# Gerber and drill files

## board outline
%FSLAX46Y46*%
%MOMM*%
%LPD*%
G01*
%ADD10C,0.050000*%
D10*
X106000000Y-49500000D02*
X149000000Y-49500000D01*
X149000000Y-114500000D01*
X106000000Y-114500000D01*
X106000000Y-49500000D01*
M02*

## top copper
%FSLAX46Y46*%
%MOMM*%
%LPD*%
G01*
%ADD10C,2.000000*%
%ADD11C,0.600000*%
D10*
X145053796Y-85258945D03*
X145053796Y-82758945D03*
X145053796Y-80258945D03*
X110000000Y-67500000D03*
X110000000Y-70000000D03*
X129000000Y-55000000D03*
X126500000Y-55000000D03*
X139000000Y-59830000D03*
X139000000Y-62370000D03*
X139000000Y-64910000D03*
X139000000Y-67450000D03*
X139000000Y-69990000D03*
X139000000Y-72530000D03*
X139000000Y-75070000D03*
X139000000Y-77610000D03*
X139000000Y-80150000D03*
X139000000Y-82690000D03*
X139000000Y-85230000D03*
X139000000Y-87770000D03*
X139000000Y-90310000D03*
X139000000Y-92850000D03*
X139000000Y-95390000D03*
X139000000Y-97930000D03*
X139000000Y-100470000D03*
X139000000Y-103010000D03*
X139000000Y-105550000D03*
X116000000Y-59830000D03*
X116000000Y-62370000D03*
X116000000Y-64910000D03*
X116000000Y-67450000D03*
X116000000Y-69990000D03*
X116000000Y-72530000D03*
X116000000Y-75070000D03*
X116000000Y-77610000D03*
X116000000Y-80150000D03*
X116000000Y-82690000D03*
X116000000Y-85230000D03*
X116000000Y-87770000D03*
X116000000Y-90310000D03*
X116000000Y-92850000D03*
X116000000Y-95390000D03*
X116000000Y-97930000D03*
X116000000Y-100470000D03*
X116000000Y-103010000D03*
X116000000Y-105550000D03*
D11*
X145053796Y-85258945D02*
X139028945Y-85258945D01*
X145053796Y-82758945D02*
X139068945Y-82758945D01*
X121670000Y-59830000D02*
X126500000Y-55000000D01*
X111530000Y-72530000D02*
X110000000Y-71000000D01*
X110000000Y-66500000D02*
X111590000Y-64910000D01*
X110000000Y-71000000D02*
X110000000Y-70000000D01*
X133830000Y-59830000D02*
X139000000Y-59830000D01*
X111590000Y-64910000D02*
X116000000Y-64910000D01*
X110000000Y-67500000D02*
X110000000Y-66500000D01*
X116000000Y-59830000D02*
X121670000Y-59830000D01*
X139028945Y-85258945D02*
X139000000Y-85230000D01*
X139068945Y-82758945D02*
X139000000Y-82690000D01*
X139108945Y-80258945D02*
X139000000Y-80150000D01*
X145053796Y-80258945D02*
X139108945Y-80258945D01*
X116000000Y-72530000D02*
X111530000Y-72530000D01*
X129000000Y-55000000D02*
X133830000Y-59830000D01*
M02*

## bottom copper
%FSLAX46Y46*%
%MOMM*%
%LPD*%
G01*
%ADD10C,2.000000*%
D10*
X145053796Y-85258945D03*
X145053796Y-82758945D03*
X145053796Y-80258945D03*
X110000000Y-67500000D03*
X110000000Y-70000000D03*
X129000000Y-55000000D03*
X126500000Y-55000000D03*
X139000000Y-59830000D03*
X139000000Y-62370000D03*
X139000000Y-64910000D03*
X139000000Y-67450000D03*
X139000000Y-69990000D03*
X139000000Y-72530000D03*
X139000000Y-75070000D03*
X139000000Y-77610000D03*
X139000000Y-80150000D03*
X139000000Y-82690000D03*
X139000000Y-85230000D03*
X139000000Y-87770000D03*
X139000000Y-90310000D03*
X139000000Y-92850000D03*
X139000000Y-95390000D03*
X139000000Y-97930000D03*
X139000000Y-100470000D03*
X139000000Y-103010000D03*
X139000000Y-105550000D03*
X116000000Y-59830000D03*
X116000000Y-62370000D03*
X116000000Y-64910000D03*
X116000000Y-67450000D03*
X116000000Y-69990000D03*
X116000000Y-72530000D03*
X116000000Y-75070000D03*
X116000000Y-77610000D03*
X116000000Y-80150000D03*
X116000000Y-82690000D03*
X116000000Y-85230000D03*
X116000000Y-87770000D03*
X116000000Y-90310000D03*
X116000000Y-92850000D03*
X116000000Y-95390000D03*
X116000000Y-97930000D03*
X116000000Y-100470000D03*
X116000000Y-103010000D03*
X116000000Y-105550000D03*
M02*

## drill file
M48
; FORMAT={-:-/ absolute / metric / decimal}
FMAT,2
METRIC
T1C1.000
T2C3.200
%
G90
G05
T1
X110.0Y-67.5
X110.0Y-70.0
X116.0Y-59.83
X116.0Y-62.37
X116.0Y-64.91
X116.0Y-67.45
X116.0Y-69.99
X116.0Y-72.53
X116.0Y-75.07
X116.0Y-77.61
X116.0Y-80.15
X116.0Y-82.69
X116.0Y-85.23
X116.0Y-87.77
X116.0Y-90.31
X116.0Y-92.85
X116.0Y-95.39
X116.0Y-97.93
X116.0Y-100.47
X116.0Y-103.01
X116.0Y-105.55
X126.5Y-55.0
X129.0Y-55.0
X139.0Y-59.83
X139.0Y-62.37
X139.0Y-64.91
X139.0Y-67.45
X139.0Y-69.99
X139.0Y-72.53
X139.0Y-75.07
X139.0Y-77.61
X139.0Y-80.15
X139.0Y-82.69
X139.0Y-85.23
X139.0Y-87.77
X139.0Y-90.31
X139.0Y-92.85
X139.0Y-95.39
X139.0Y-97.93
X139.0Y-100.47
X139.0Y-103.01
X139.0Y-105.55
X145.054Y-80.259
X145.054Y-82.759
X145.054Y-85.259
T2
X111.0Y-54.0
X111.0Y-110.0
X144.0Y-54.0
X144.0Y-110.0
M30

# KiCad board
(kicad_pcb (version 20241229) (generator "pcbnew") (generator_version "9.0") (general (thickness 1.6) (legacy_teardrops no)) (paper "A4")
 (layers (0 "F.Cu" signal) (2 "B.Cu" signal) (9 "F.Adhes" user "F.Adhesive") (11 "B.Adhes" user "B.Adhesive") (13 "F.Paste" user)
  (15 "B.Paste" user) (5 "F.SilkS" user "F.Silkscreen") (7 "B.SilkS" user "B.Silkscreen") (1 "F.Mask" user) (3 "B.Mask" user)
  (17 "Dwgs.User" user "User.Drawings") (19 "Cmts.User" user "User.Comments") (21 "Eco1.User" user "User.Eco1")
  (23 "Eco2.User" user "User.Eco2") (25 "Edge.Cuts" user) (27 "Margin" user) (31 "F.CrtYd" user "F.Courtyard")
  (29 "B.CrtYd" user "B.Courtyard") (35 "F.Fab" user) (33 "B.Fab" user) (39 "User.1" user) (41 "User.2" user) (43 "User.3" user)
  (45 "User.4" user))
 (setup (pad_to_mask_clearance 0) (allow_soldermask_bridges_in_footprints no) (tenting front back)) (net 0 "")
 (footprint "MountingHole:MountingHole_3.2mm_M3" (layer "F.Cu") (at 144 110)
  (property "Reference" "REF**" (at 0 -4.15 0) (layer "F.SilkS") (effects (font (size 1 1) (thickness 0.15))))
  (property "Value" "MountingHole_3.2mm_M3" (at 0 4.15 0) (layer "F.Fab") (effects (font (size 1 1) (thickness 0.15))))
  (pad "" np_thru_hole circle (at 0 0) (size 3.2 3.2) (drill 3.2) (layers "*.Cu" "*.Mask")))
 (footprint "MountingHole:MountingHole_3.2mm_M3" (layer "F.Cu") (at 144 54)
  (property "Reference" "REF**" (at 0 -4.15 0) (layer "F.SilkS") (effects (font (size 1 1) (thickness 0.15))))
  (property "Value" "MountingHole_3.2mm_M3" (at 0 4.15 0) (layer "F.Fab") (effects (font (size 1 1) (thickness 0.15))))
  (pad "" np_thru_hole circle (at 0 0) (size 3.2 3.2) (drill 3.2) (layers "*.Cu" "*.Mask")))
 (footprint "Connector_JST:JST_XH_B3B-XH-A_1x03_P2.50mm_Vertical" (layer "F.Cu") (at 145.053796 85.258945 90)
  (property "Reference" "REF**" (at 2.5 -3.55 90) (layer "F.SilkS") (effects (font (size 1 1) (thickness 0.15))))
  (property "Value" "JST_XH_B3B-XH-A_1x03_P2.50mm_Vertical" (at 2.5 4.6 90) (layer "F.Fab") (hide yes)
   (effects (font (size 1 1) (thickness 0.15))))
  (pad "1" thru_hole circle (at 0 0 90) (size 2 2) (drill 1) (layers "*.Cu" "*.Mask") (remove_unused_layers no))
  (pad "2" thru_hole circle (at 2.5 0 90) (size 2 2) (drill 1) (layers "*.Cu" "*.Mask") (remove_unused_layers no))
  (pad "3" thru_hole circle (at 5 0 90) (size 2 2) (drill 1) (layers "*.Cu" "*.Mask") (remove_unused_layers no)))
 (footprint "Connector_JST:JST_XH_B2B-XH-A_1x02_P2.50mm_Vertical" (layer "F.Cu") (at 110 67.5 -90)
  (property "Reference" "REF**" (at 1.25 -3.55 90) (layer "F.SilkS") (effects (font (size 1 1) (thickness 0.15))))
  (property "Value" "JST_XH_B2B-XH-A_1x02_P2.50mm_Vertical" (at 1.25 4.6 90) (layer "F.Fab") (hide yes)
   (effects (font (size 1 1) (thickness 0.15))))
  (pad "1" thru_hole circle (at 0 0 270) (size 2 2) (drill 1) (layers "*.Cu" "*.Mask") (remove_unused_layers no))
  (pad "2" thru_hole circle (at 2.5 0 270) (size 2 2) (drill 1) (layers "*.Cu" "*.Mask") (remove_unused_layers no)))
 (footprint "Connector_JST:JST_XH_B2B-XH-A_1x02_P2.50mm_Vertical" (layer "F.Cu") (at 129 55 180)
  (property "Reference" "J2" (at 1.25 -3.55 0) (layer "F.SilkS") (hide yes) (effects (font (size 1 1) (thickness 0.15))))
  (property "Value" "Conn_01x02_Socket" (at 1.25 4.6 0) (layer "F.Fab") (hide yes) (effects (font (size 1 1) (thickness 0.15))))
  (pad "1" thru_hole circle (at 0 0 180) (size 2 2) (drill 1) (layers "*.Cu" "*.Mask") (remove_unused_layers no))
  (pad "2" thru_hole circle (at 2.5 0 180) (size 2 2) (drill 1) (layers "*.Cu" "*.Mask") (remove_unused_layers no)))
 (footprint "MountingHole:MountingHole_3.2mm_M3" (layer "F.Cu") (at 111 110)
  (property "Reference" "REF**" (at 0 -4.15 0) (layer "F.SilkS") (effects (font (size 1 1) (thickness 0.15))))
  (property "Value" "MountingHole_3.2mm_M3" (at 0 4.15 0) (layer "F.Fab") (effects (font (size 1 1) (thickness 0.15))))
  (pad "" np_thru_hole circle (at 0 0) (size 3.2 3.2) (drill 3.2) (layers "*.Cu" "*.Mask")))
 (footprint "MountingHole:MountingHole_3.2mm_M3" (layer "F.Cu") (at 111 54)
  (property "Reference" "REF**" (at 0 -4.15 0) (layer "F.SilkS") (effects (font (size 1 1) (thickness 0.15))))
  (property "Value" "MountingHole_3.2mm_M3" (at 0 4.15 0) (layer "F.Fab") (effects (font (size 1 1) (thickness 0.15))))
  (pad "" np_thru_hole circle (at 0 0) (size 3.2 3.2) (drill 3.2) (layers "*.Cu" "*.Mask")))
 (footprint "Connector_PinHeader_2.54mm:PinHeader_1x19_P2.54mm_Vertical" (layer "B.Cu") (at 139 59.83 180)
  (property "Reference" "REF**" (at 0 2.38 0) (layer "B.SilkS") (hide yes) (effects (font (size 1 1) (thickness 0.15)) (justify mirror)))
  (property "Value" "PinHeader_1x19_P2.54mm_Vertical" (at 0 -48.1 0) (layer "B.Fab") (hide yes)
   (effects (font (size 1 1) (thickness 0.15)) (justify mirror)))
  (pad "1" thru_hole circle (at 0 0 180) (size 2 2) (drill 1) (layers "*.Cu" "*.Mask") (remove_unused_layers no))
  (pad "2" thru_hole circle (at 0 -2.54 180) (size 2 2) (drill 1) (layers "*.Cu" "*.Mask") (remove_unused_layers no))
  (pad "3" thru_hole circle (at 0 -5.08 180) (size 2 2) (drill 1) (layers "*.Cu" "*.Mask") (remove_unused_layers no))
  (pad "4" thru_hole circle (at 0 -7.62 180) (size 2 2) (drill 1) (layers "*.Cu" "*.Mask") (remove_unused_layers no))
  (pad "5" thru_hole circle (at 0 -10.16 180) (size 2 2) (drill 1) (layers "*.Cu" "*.Mask") (remove_unused_layers no))
  (pad "6" thru_hole circle (at 0 -12.7 180) (size 2 2) (drill 1) (layers "*.Cu" "*.Mask") (remove_unused_layers no))
  (pad "7" thru_hole circle (at 0 -15.24 180) (size 2 2) (drill 1) (layers "*.Cu" "*.Mask") (remove_unused_layers no))
  (pad "8" thru_hole circle (at 0 -17.78 180) (size 2 2) (drill 1) (layers "*.Cu" "*.Mask") (remove_unused_layers no))
  (pad "9" thru_hole circle (at 0 -20.32 180) (size 2 2) (drill 1) (layers "*.Cu" "*.Mask") (remove_unused_layers no))
  (pad "10" thru_hole circle (at 0 -22.86 180) (size 2 2) (drill 1) (layers "*.Cu" "*.Mask") (remove_unused_layers no))
  (pad "11" thru_hole circle (at 0 -25.4 180) (size 2 2) (drill 1) (layers "*.Cu" "*.Mask") (remove_unused_layers no))
  (pad "12" thru_hole circle (at 0 -27.94 180) (size 2 2) (drill 1) (layers "*.Cu" "*.Mask") (remove_unused_layers no))
  (pad "13" thru_hole circle (at 0 -30.48 180) (size 2 2) (drill 1) (layers "*.Cu" "*.Mask") (remove_unused_layers no))
  (pad "14" thru_hole circle (at 0 -33.02 180) (size 2 2) (drill 1) (layers "*.Cu" "*.Mask") (remove_unused_layers no))
  (pad "15" thru_hole circle (at 0 -35.56 180) (size 2 2) (drill 1) (layers "*.Cu" "*.Mask") (remove_unused_layers no))
  (pad "16" thru_hole circle (at 0 -38.1 180) (size 2 2) (drill 1) (layers "*.Cu" "*.Mask") (remove_unused_layers no))
  (pad "17" thru_hole circle (at 0 -40.64 180) (size 2 2) (drill 1) (layers "*.Cu" "*.Mask") (remove_unused_layers no))
  (pad "18" thru_hole circle (at 0 -43.18 180) (size 2 2) (drill 1) (layers "*.Cu" "*.Mask") (remove_unused_layers no))
  (pad "19" thru_hole circle (at 0 -45.72 180) (size 2 2) (drill 1) (layers "*.Cu" "*.Mask") (remove_unused_layers no)))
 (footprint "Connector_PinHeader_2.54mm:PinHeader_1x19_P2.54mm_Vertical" (layer "B.Cu") (at 116 59.83 180)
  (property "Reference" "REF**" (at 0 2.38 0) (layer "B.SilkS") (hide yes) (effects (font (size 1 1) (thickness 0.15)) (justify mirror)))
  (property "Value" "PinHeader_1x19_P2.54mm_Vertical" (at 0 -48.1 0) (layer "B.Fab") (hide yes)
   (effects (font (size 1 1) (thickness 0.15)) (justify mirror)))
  (pad "1" thru_hole circle (at 0 0 180) (size 2 2) (drill 1) (layers "*.Cu" "*.Mask") (remove_unused_layers no))
  (pad "2" thru_hole circle (at 0 -2.54 180) (size 2 2) (drill 1) (layers "*.Cu" "*.Mask") (remove_unused_layers no))
  (pad "3" thru_hole circle (at 0 -5.08 180) (size 2 2) (drill 1) (layers "*.Cu" "*.Mask") (remove_unused_layers no))
  (pad "4" thru_hole circle (at 0 -7.62 180) (size 2 2) (drill 1) (layers "*.Cu" "*.Mask") (remove_unused_layers no))
  (pad "5" thru_hole circle (at 0 -10.16 180) (size 2 2) (drill 1) (layers "*.Cu" "*.Mask") (remove_unused_layers no))
  (pad "6" thru_hole circle (at 0 -12.7 180) (size 2 2) (drill 1) (layers "*.Cu" "*.Mask") (remove_unused_layers no))
  (pad "7" thru_hole circle (at 0 -15.24 180) (size 2 2) (drill 1) (layers "*.Cu" "*.Mask") (remove_unused_layers no))
  (pad "8" thru_hole circle (at 0 -17.78 180) (size 2 2) (drill 1) (layers "*.Cu" "*.Mask") (remove_unused_layers no))
  (pad "9" thru_hole circle (at 0 -20.32 180) (size 2 2) (drill 1) (layers "*.Cu" "*.Mask") (remove_unused_layers no))
  (pad "10" thru_hole circle (at 0 -22.86 180) (size 2 2) (drill 1) (layers "*.Cu" "*.Mask") (remove_unused_layers no))
  (pad "11" thru_hole circle (at 0 -25.4 180) (size 2 2) (drill 1) (layers "*.Cu" "*.Mask") (remove_unused_layers no))
  (pad "12" thru_hole circle (at 0 -27.94 180) (size 2 2) (drill 1) (layers "*.Cu" "*.Mask") (remove_unused_layers no))
  (pad "13" thru_hole circle (at 0 -30.48 180) (size 2 2) (drill 1) (layers "*.Cu" "*.Mask") (remove_unused_layers no))
  (pad "14" thru_hole circle (at 0 -33.02 180) (size 2 2) (drill 1) (layers "*.Cu" "*.Mask") (remove_unused_layers no))
  (pad "15" thru_hole circle (at 0 -35.56 180) (size 2 2) (drill 1) (layers "*.Cu" "*.Mask") (remove_unused_layers no))
  (pad "16" thru_hole circle (at 0 -38.1 180) (size 2 2) (drill 1) (layers "*.Cu" "*.Mask") (remove_unused_layers no))
  (pad "17" thru_hole circle (at 0 -40.64 180) (size 2 2) (drill 1) (layers "*.Cu" "*.Mask") (remove_unused_layers no))
  (pad "18" thru_hole circle (at 0 -43.18 180) (size 2 2) (drill 1) (layers "*.Cu" "*.Mask") (remove_unused_layers no))
  (pad "19" thru_hole circle (at 0 -45.72 180) (size 2 2) (drill 1) (layers "*.Cu" "*.Mask") (remove_unused_layers no)))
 (gr_rect (start 106 49.5) (end 149 114.5) (stroke (width 0.05) (type default)) (fill no) (layer "Edge.Cuts"))
 (segment (start 145.053796 85.258945) (end 139.028945 85.258945) (width 0.6) (layer "F.Cu") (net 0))
 (segment (start 145.053796 82.758945) (end 139.068945 82.758945) (width 0.6) (layer "F.Cu") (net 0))
 (segment (start 121.67 59.83) (end 126.5 55) (width 0.6) (layer "F.Cu") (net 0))
 (segment (start 111.53 72.53) (end 110 71) (width 0.6) (layer "F.Cu") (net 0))
 (segment (start 110 66.5) (end 111.59 64.91) (width 0.6) (layer "F.Cu") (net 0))
 (segment (start 110 71) (end 110 70) (width 0.6) (layer "F.Cu") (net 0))
 (segment (start 133.83 59.83) (end 139 59.83) (width 0.6) (layer "F.Cu") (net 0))
 (segment (start 111.59 64.91) (end 116 64.91) (width 0.6) (layer "F.Cu") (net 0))
 (segment (start 110 67.5) (end 110 66.5) (width 0.6) (layer "F.Cu") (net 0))
 (segment (start 116 59.83) (end 121.67 59.83) (width 0.6) (layer "F.Cu") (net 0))
 (segment (start 139.028945 85.258945) (end 139 85.23) (width 0.6) (layer "F.Cu") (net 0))
 (segment (start 139.068945 82.758945) (end 139 82.69) (width 0.6) (layer "F.Cu") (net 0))
 (segment (start 139.108945 80.258945) (end 139 80.15) (width 0.6) (layer "F.Cu") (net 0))
 (segment (start 145.053796 80.258945) (end 139.108945 80.258945) (width 0.6) (layer "F.Cu") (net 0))
 (segment (start 116 72.53) (end 111.53 72.53) (width 0.6) (layer "F.Cu") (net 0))
 (segment (start 129 55) (end 133.83 59.83) (width 0.6) (layer "F.Cu") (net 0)))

